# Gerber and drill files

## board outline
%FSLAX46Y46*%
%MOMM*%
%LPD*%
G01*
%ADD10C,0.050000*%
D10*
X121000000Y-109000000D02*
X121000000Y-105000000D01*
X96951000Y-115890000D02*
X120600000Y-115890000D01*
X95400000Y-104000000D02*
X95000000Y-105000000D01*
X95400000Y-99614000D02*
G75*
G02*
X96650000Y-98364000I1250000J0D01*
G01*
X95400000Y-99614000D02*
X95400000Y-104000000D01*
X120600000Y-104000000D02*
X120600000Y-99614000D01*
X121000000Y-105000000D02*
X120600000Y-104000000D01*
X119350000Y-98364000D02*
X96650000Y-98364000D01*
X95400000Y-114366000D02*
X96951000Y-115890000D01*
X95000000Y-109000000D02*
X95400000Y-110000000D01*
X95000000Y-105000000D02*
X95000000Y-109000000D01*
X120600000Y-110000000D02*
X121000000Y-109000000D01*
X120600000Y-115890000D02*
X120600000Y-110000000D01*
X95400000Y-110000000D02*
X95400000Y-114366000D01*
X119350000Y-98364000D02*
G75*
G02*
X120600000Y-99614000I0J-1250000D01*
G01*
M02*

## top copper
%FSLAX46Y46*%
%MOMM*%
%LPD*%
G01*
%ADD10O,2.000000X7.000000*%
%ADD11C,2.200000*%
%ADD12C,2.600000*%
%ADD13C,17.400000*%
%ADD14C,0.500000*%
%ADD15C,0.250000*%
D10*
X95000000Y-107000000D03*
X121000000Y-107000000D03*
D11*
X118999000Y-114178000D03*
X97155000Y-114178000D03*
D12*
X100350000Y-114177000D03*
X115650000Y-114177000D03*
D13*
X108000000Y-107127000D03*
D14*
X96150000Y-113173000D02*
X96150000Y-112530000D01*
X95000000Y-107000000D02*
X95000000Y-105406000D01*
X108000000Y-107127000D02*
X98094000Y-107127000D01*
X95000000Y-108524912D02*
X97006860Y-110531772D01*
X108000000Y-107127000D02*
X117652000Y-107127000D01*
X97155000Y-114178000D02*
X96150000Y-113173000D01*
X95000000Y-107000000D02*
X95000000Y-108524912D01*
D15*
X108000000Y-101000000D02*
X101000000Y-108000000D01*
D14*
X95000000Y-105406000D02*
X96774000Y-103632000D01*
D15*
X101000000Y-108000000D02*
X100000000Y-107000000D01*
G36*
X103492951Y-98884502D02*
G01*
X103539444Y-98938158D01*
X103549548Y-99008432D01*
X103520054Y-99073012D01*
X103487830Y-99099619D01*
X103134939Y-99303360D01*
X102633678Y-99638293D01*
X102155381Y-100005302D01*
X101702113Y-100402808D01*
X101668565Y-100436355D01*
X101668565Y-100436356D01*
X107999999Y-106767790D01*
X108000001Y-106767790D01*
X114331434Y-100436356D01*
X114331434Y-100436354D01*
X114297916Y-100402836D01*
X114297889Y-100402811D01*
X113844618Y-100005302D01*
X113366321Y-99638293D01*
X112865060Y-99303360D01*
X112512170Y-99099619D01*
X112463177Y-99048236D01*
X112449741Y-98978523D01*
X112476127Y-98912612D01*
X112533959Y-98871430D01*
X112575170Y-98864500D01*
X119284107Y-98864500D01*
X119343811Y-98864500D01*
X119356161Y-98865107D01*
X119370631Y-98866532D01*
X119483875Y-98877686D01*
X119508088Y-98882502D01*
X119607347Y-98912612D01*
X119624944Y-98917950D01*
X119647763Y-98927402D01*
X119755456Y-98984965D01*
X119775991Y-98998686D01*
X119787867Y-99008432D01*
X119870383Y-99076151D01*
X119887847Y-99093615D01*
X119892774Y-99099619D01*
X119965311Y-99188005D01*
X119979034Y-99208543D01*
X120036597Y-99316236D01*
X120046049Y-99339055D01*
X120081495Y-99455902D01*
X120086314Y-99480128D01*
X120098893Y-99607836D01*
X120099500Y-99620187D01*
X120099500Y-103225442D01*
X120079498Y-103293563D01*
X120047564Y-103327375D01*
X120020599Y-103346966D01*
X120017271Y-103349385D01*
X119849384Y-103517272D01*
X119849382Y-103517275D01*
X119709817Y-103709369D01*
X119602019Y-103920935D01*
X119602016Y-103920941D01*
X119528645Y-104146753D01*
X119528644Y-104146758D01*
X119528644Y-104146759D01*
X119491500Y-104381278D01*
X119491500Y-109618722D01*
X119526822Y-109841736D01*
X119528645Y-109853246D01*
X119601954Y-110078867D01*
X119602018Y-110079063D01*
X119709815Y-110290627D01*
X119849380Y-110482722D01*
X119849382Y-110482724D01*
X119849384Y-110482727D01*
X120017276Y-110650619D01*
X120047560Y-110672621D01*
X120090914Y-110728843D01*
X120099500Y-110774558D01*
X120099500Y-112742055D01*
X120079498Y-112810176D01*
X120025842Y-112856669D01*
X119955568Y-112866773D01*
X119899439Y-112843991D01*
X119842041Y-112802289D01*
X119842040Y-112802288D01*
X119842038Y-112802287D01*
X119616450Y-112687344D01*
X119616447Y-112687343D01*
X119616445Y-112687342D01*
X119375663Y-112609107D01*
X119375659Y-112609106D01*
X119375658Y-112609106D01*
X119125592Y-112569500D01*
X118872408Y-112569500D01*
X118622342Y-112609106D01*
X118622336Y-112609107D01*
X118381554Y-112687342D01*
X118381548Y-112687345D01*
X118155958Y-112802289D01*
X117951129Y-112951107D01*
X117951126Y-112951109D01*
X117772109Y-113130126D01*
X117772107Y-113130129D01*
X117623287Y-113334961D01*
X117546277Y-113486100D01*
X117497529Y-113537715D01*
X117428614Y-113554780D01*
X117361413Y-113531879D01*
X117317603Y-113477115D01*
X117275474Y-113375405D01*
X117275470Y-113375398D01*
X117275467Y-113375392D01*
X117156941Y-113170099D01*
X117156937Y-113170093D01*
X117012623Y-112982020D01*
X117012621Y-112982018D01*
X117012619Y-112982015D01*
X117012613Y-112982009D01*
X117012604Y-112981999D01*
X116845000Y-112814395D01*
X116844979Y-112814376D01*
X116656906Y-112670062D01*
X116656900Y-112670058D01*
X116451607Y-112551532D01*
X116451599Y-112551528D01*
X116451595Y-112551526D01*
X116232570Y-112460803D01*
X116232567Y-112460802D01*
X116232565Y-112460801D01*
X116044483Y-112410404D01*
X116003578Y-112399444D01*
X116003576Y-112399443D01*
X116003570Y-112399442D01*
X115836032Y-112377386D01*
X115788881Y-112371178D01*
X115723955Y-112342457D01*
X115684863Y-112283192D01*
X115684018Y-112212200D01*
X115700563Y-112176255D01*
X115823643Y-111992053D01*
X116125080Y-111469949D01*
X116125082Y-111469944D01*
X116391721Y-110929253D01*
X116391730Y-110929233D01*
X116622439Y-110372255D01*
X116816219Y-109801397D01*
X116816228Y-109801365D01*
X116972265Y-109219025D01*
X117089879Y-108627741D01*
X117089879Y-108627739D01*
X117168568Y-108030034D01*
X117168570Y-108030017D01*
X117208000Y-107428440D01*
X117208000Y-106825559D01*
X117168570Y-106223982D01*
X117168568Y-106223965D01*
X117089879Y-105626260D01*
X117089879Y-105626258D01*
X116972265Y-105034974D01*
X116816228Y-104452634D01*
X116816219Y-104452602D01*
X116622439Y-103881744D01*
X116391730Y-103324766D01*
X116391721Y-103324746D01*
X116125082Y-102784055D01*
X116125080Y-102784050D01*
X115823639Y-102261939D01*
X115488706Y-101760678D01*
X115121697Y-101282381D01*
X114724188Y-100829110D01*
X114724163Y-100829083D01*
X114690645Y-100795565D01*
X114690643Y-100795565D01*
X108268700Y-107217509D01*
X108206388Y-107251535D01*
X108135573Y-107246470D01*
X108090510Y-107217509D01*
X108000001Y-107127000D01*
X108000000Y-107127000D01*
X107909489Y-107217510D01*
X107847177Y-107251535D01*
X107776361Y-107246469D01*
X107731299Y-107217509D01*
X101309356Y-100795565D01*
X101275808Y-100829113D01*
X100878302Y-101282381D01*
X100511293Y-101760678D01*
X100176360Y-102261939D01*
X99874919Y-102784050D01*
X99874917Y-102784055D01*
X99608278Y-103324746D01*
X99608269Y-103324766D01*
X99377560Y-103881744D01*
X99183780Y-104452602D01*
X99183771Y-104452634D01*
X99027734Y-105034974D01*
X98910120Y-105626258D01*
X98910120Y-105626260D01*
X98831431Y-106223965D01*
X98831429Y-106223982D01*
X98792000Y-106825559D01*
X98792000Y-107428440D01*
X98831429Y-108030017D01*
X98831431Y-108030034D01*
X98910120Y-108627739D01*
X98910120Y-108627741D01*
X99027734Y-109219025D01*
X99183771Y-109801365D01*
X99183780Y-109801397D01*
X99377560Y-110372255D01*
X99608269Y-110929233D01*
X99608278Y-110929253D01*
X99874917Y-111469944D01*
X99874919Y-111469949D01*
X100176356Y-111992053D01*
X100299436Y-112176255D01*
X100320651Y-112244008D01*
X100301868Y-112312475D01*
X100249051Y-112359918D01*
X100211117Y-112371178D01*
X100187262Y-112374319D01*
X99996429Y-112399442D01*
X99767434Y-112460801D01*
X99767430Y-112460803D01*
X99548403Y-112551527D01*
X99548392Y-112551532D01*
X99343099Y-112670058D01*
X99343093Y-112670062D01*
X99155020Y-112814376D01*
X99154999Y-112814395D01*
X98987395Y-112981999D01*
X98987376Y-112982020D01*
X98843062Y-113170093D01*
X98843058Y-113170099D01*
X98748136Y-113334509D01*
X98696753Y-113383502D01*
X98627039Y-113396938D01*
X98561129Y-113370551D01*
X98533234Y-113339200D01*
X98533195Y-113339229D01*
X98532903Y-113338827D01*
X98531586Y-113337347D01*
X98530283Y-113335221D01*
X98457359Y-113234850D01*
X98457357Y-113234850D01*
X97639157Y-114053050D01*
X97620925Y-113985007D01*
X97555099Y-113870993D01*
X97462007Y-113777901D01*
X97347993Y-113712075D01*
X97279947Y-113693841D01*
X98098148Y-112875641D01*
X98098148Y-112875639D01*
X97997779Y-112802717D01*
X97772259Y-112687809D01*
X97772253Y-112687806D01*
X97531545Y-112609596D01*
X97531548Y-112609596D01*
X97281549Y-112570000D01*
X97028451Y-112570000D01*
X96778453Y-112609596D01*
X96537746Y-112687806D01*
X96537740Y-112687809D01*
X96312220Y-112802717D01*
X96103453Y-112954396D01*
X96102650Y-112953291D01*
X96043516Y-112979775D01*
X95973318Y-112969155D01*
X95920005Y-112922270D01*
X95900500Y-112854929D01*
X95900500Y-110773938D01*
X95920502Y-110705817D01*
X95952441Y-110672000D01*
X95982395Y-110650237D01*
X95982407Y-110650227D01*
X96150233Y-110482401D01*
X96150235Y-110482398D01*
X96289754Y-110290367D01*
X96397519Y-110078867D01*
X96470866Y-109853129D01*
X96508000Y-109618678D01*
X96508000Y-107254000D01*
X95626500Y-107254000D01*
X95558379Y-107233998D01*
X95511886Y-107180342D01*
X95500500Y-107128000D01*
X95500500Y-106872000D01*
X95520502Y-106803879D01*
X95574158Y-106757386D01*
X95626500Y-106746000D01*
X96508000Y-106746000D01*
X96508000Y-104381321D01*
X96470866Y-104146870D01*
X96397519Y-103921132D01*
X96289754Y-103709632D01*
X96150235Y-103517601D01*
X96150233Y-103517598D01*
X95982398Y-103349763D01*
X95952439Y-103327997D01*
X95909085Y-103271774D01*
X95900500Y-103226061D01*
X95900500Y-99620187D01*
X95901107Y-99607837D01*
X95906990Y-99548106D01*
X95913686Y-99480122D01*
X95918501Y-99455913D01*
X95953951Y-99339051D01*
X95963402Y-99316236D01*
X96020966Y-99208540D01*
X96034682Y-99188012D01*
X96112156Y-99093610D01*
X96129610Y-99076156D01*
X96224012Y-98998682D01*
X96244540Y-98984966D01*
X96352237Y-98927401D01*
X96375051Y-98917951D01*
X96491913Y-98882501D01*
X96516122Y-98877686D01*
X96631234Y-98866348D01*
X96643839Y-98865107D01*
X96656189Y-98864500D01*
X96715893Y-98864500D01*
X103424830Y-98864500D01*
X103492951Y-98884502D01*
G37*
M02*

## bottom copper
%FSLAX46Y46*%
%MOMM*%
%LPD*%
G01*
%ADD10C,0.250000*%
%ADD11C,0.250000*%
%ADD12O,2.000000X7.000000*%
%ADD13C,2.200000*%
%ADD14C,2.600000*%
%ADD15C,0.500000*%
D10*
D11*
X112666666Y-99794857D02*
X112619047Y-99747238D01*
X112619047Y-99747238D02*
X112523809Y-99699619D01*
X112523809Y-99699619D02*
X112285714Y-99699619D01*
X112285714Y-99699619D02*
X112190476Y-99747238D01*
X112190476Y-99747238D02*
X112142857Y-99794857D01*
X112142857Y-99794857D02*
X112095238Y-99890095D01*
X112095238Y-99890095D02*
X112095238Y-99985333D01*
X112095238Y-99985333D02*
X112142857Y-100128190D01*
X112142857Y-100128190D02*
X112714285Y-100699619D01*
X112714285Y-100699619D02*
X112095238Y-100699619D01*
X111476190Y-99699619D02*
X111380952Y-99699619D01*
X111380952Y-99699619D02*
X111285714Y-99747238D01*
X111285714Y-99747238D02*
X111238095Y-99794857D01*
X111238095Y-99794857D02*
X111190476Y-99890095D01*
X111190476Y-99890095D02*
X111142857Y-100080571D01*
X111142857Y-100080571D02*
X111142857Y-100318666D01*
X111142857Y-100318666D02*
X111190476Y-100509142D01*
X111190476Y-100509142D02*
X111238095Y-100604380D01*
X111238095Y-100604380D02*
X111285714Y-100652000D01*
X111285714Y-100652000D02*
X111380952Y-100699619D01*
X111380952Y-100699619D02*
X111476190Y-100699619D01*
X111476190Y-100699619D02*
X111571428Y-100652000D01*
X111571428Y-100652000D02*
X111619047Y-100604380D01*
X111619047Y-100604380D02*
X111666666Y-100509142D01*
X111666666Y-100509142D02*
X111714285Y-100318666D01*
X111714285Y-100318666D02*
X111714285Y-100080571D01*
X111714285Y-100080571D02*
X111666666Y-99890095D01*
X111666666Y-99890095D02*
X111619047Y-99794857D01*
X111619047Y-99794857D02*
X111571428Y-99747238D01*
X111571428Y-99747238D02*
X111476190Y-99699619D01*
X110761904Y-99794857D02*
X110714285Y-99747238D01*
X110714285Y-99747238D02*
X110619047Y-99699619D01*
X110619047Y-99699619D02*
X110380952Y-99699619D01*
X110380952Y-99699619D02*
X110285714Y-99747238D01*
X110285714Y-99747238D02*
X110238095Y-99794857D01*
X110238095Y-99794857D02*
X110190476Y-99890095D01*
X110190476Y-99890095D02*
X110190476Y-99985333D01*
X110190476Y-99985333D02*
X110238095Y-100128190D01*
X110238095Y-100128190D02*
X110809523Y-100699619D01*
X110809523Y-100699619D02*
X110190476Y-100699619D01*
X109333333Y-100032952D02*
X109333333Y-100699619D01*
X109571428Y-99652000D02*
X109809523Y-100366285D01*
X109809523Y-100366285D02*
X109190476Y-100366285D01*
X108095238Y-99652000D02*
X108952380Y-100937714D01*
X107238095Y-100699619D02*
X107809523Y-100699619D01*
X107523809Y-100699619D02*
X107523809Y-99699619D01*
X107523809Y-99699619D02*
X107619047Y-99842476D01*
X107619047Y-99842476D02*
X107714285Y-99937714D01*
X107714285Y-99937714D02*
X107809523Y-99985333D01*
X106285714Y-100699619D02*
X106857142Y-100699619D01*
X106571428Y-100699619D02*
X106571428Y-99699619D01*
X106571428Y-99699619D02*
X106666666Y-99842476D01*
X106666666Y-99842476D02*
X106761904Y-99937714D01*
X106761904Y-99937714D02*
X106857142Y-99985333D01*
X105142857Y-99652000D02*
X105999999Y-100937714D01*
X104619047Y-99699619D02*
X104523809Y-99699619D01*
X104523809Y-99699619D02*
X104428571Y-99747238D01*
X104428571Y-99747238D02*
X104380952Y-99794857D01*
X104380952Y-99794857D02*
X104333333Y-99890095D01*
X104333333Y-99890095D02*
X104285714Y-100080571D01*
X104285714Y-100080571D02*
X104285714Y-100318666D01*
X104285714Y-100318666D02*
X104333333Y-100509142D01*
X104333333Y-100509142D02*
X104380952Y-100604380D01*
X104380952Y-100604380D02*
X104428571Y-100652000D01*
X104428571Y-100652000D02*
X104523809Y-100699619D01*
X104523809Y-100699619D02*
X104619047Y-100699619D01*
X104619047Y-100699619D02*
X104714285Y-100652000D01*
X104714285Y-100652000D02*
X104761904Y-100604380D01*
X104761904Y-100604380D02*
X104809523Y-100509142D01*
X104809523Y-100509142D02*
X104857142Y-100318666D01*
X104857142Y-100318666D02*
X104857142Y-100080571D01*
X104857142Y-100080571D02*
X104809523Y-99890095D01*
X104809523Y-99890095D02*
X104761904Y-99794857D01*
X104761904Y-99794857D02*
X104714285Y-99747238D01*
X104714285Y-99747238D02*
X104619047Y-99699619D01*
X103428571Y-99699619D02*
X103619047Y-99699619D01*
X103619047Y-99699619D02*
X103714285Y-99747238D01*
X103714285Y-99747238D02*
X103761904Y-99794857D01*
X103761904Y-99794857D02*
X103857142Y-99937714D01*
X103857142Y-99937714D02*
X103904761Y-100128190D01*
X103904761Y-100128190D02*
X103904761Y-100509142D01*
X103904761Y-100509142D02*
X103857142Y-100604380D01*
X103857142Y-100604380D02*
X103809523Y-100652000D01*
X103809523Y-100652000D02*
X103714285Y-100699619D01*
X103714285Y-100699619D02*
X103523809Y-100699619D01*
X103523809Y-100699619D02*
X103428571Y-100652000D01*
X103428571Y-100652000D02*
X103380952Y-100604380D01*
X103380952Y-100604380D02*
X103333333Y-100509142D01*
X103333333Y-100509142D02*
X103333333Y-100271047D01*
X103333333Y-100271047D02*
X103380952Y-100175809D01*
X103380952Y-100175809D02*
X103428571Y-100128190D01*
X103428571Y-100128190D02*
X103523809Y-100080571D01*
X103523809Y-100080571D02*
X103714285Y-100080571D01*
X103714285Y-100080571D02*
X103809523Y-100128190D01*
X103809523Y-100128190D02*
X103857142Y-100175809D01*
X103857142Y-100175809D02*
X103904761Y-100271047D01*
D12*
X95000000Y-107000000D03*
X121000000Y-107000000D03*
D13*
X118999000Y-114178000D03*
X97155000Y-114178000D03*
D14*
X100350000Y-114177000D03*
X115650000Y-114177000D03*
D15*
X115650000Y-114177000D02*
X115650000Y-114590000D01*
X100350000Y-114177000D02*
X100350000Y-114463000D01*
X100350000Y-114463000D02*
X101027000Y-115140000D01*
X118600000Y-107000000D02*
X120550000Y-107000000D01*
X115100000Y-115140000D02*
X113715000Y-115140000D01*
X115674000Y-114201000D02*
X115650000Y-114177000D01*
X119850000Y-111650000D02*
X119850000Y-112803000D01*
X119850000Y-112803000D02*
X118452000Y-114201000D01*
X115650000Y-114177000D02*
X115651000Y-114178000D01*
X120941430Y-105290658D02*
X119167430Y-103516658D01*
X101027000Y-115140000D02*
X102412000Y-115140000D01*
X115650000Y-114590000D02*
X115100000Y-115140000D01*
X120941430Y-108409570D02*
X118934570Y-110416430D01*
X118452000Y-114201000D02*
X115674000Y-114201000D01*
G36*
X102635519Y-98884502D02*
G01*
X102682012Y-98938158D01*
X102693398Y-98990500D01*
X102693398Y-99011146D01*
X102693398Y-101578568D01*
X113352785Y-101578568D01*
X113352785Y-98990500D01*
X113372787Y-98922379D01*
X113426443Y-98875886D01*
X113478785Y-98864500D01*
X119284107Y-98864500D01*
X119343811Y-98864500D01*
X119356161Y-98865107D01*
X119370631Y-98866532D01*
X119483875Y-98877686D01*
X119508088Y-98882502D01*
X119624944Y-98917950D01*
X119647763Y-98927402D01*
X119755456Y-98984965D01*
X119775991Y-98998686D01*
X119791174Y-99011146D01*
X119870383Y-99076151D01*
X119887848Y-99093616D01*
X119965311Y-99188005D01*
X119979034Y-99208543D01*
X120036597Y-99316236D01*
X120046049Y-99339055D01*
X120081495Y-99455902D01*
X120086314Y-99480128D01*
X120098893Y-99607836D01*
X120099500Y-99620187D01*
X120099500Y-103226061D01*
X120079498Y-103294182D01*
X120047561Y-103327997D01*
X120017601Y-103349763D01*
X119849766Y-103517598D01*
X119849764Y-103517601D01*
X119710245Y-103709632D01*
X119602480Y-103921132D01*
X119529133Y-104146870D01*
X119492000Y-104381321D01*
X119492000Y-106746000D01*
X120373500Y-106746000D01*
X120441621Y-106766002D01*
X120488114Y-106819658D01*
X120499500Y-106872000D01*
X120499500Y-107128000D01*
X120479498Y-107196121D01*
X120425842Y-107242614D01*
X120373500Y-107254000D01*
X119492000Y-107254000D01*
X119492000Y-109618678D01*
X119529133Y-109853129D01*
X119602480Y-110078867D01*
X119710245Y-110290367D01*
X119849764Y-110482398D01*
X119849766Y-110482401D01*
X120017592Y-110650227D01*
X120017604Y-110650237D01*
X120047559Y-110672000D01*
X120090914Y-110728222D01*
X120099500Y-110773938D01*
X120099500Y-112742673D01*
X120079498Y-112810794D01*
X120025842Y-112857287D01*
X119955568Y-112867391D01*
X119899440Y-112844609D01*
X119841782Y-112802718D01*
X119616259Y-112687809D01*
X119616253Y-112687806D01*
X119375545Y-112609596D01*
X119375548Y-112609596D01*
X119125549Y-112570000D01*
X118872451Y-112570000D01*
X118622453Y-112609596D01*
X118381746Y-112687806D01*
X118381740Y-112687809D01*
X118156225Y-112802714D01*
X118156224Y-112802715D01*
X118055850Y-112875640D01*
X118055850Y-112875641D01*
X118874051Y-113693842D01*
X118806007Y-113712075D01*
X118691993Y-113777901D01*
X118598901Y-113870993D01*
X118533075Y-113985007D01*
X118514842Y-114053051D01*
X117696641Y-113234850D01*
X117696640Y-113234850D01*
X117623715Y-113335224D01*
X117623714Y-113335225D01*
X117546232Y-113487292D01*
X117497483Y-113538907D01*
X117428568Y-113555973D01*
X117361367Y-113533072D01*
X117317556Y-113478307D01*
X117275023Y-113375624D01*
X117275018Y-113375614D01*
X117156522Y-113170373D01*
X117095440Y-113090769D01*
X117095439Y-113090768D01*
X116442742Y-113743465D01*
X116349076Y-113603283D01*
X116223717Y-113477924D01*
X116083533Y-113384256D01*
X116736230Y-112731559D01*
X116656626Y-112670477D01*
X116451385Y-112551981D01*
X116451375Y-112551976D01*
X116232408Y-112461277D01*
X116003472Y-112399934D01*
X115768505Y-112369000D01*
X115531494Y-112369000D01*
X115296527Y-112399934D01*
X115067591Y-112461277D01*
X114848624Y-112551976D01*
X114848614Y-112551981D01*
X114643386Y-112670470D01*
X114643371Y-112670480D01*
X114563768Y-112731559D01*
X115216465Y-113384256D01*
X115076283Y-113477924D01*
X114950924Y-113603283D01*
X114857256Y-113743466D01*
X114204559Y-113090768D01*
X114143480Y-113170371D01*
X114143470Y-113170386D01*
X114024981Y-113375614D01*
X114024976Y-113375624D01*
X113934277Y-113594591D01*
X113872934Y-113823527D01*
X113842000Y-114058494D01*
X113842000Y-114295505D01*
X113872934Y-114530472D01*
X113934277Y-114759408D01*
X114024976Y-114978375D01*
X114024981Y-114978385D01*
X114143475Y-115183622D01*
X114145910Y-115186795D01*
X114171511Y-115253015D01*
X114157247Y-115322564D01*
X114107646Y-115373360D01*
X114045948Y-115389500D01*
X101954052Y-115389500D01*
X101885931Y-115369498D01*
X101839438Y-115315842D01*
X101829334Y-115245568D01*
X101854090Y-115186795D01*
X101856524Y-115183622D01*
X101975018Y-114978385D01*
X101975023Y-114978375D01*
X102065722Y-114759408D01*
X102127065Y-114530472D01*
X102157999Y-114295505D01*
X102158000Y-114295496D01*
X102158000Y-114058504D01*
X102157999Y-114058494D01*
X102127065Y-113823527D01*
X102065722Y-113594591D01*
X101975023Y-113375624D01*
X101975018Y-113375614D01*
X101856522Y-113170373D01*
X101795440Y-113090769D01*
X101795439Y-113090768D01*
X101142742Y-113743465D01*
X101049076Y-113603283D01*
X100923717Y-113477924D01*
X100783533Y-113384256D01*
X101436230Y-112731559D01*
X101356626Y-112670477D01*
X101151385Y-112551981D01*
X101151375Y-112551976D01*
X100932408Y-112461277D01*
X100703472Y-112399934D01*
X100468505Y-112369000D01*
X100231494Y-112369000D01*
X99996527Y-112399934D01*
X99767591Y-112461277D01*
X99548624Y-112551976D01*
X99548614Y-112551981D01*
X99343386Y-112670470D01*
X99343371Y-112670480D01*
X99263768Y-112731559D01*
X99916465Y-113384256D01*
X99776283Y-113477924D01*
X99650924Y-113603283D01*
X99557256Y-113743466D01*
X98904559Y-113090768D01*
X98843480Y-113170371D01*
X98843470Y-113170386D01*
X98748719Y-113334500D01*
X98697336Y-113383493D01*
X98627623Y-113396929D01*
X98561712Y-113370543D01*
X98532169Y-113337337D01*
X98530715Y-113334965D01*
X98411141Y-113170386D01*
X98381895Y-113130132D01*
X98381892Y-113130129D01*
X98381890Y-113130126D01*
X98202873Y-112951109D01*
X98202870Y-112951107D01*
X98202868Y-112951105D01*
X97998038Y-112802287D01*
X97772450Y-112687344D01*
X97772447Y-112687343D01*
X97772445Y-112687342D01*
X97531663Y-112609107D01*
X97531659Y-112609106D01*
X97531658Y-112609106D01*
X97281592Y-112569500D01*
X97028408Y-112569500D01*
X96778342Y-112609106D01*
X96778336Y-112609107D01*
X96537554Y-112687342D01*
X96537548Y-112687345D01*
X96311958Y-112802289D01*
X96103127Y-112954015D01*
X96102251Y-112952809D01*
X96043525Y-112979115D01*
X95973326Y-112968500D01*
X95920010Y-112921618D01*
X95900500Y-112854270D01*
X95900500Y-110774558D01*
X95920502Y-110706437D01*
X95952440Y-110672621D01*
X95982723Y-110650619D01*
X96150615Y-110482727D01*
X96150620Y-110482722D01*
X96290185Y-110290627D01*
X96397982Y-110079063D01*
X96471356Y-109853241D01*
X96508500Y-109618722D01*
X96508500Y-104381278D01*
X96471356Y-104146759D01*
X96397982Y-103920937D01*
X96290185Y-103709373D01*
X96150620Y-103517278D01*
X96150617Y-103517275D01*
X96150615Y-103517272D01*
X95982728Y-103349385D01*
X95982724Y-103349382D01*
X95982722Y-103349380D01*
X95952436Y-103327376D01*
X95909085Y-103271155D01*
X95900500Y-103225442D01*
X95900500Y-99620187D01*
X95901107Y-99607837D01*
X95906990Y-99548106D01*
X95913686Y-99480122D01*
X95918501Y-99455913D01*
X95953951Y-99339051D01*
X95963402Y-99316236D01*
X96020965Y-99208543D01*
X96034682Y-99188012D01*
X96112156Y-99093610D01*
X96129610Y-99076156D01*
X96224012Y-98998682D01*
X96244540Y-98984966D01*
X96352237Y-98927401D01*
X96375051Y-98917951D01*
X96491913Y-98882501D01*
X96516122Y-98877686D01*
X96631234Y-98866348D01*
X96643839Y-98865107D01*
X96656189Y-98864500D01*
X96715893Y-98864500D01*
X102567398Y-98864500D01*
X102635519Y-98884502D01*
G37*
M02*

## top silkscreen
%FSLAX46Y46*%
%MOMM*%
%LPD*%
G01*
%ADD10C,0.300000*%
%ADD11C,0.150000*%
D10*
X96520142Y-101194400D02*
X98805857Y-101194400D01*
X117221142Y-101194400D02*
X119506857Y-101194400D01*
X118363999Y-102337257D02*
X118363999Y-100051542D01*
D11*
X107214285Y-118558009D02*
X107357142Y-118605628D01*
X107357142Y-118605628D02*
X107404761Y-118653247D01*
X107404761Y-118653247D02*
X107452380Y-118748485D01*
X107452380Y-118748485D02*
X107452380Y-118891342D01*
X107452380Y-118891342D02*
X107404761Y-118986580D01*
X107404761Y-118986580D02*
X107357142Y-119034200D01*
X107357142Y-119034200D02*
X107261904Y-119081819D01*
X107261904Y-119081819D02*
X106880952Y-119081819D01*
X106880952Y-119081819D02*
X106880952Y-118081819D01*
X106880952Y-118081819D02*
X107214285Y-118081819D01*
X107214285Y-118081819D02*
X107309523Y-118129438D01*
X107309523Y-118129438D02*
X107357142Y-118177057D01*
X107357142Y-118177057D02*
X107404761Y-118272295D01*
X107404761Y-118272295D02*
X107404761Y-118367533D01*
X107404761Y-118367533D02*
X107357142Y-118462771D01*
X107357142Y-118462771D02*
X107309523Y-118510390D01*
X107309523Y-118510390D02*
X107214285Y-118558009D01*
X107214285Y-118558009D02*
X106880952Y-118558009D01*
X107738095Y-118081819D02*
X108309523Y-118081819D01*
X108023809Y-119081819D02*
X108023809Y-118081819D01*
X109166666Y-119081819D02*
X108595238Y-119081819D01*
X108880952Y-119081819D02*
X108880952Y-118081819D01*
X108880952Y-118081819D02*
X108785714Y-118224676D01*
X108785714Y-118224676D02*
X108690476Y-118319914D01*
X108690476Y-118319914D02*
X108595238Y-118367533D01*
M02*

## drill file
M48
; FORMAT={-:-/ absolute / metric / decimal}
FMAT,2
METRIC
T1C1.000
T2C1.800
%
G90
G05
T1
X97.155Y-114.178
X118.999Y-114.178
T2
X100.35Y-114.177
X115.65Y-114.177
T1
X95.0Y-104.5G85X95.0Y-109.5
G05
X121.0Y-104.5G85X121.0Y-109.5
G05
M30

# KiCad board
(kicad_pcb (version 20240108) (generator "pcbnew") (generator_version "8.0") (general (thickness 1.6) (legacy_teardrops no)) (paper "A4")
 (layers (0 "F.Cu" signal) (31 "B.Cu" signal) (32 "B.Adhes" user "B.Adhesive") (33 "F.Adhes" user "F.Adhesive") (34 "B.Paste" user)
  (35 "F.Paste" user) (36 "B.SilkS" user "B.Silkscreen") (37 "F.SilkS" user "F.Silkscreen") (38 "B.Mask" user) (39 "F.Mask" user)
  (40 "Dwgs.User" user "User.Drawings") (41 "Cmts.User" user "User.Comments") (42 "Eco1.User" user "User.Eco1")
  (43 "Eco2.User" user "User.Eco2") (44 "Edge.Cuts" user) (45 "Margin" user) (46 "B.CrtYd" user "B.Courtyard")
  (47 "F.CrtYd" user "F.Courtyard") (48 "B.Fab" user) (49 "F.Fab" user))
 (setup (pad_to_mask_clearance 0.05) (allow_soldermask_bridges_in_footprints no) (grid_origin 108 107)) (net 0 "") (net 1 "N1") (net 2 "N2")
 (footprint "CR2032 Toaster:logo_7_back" (layer "F.Cu") (at 114 106.25)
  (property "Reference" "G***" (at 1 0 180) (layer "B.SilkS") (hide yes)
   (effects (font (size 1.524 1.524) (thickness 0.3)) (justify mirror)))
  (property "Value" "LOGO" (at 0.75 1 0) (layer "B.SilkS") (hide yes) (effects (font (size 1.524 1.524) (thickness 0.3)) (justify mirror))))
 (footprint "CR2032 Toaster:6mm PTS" (layer "F.Cu") (at 95 107)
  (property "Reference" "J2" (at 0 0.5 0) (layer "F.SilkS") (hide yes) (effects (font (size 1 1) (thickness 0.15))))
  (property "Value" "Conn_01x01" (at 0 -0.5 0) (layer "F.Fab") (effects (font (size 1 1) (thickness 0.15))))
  (pad "1" thru_hole oval (at 0 0) (size 2 7) (drill oval 1 6) (layers "*.Cu" "*.Mask") (remove_unused_layers no) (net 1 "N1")))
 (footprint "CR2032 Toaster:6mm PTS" (layer "F.Cu") (at 121 107)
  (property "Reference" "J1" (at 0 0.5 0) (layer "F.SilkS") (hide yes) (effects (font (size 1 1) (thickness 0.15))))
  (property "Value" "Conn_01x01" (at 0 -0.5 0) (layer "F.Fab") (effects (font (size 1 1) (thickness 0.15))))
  (pad "1" thru_hole oval (at 0 0) (size 2 7) (drill oval 1 6) (layers "*.Cu" "*.Mask") (remove_unused_layers no) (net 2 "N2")))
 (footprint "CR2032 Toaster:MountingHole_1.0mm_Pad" (layer "F.Cu") (at 118.999 114.178)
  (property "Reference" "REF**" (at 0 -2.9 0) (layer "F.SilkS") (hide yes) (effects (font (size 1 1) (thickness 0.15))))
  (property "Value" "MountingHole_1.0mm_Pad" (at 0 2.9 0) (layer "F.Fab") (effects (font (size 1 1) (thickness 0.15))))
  (pad "1" thru_hole circle (at 0 0) (size 2.2 2.2) (drill 1) (layers "*.Cu" "*.Mask") (remove_unused_layers no) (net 2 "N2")))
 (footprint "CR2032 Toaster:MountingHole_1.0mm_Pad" (layer "F.Cu") (at 97.155 114.178)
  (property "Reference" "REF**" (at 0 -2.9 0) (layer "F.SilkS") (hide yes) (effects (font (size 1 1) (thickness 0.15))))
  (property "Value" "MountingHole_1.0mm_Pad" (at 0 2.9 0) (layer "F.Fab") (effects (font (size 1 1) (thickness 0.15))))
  (pad "1" thru_hole circle (at 0 0) (size 2.2 2.2) (drill 1) (layers "*.Cu" "*.Mask") (remove_unused_layers no) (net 1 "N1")))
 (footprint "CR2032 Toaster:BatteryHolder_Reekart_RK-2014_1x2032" (layer "F.Cu") (at 108 107.127)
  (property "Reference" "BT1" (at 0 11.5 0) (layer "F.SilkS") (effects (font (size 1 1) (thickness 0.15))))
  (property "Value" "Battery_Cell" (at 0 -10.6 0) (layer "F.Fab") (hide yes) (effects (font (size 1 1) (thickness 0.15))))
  (pad "1" thru_hole circle (at -7.65 7.05) (size 2.6 2.6) (drill 1.8) (layers "*.Cu" "*.Mask") (remove_unused_layers no) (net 2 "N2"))
  (pad "1" thru_hole circle (at 7.65 7.05) (size 2.6 2.6) (drill 1.8) (layers "*.Cu" "*.Mask") (remove_unused_layers no) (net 2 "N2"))
  (pad "2" smd circle (at 0 0) (size 17.4 17.4) (layers "F.Cu" "F.Paste" "F.Mask") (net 1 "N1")))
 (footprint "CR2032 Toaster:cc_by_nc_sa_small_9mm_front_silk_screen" (layer "B.Cu") (at 107.95 113.5 180)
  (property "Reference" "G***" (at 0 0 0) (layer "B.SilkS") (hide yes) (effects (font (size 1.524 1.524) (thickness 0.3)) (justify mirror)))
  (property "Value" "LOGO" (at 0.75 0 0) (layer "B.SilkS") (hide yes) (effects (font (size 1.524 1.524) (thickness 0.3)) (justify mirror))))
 (gr_line (start 121 109) (end 121 105) (stroke (width 0.05) (type solid)) (layer "Edge.Cuts"))
 (gr_line (start 96.951 115.89) (end 120.6 115.89) (stroke (width 0.05) (type solid)) (layer "Edge.Cuts"))
 (gr_line (start 95.4 104) (end 95 105) (stroke (width 0.05) (type solid)) (layer "Edge.Cuts"))
 (gr_arc (start 95.4 99.614) (mid 95.766117 98.730117) (end 96.65 98.364) (stroke (width 0.05) (type solid)) (layer "Edge.Cuts"))
 (gr_line (start 95.4 99.614) (end 95.4 104) (stroke (width 0.05) (type solid)) (layer "Edge.Cuts"))
 (gr_line (start 120.6 104) (end 120.6 99.614) (stroke (width 0.05) (type solid)) (layer "Edge.Cuts"))
 (gr_line (start 121 105) (end 120.6 104) (stroke (width 0.05) (type solid)) (layer "Edge.Cuts"))
 (gr_line (start 119.35 98.364) (end 96.65 98.364) (stroke (width 0.05) (type solid)) (layer "Edge.Cuts"))
 (gr_line (start 95.4 114.366) (end 96.951 115.89) (stroke (width 0.05) (type solid)) (layer "Edge.Cuts"))
 (gr_line (start 95 109) (end 95.4 110) (stroke (width 0.05) (type solid)) (layer "Edge.Cuts"))
 (gr_line (start 95 105) (end 95 109) (stroke (width 0.05) (type solid)) (layer "Edge.Cuts"))
 (gr_line (start 120.6 110) (end 121 109) (stroke (width 0.05) (type solid)) (layer "Edge.Cuts"))
 (gr_line (start 120.6 115.89) (end 120.6 110) (stroke (width 0.05) (type solid)) (layer "Edge.Cuts"))
 (gr_line (start 95.4 110) (end 95.4 114.366) (stroke (width 0.05) (type solid)) (layer "Edge.Cuts"))
 (gr_arc (start 119.35 98.364) (mid 120.233883 98.730117) (end 120.6 99.614) (stroke (width 0.05) (type solid)) (layer "Edge.Cuts"))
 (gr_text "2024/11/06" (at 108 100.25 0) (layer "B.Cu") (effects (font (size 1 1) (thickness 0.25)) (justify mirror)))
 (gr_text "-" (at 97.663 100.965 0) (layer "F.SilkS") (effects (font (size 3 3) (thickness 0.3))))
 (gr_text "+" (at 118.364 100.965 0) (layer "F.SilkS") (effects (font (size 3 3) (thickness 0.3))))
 (segment (start 115.65 114.177) (end 115.65 114.59) (width 0.5) (layer "B.Cu") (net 2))
 (segment (start 100.35 114.177) (end 100.35 114.463) (width 0.5) (layer "B.Cu") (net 2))
 (segment (start 100.35 114.463) (end 101.027 115.14) (width 0.5) (layer "B.Cu") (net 2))
 (segment (start 118.6 107) (end 120.55 107) (width 0.5) (layer "B.Cu") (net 2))
 (segment (start 115.1 115.14) (end 113.715 115.14) (width 0.5) (layer "B.Cu") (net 2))
 (segment (start 115.674 114.201) (end 115.65 114.177) (width 0.5) (layer "B.Cu") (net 2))
 (segment (start 119.85 111.65) (end 119.85 112.803) (width 0.5) (layer "B.Cu") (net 2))
 (segment (start 119.85 112.803) (end 118.452 114.201) (width 0.5) (layer "B.Cu") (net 2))
 (segment (start 115.65 114.177) (end 115.651 114.178) (width 0.5) (layer "B.Cu") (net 2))
 (segment (start 120.94143 105.290658) (end 119.16743 103.516658) (width 0.5) (layer "B.Cu") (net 2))
 (segment (start 101.027 115.14) (end 102.412 115.14) (width 0.5) (layer "B.Cu") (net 2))
 (segment (start 115.65 114.59) (end 115.1 115.14) (width 0.5) (layer "B.Cu") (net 2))
 (segment (start 120.94143 108.40957) (end 118.93457 110.41643) (width 0.5) (layer "B.Cu") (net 2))
 (segment (start 118.452 114.201) (end 115.674 114.201) (width 0.5) (layer "B.Cu") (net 2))
 (segment (start 96.15 113.173) (end 96.15 112.53) (width 0.5) (layer "F.Cu") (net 1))
 (segment (start 95 107) (end 95 105.406) (width 0.5) (layer "F.Cu") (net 1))
 (segment (start 108 107.127) (end 98.094 107.127) (width 0.5) (layer "F.Cu") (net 1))
 (segment (start 95 108.524912) (end 97.00686 110.531772) (width 0.5) (layer "F.Cu") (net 1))
 (segment (start 108 107.127) (end 117.652 107.127) (width 0.5) (layer "F.Cu") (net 1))
 (segment (start 97.155 114.178) (end 96.15 113.173) (width 0.5) (layer "F.Cu") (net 1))
 (segment (start 95 107) (end 95 108.524912) (width 0.5) (layer "F.Cu") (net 1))
 (segment (start 108 101) (end 101 108) (width 0.25) (layer "F.Cu") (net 1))
 (segment (start 95 105.406) (end 96.774 103.632) (width 0.5) (layer "F.Cu") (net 1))
 (segment (start 101 108) (end 100 107) (width 0.25) (layer "F.Cu") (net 1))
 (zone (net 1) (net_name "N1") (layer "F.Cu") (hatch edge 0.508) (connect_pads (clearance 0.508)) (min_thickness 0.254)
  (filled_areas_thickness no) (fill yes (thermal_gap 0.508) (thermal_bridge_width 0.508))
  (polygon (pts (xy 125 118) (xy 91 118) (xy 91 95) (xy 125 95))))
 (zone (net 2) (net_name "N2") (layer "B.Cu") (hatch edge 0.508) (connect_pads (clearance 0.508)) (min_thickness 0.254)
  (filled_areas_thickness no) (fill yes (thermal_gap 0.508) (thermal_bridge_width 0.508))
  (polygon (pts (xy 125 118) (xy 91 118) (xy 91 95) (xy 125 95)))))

